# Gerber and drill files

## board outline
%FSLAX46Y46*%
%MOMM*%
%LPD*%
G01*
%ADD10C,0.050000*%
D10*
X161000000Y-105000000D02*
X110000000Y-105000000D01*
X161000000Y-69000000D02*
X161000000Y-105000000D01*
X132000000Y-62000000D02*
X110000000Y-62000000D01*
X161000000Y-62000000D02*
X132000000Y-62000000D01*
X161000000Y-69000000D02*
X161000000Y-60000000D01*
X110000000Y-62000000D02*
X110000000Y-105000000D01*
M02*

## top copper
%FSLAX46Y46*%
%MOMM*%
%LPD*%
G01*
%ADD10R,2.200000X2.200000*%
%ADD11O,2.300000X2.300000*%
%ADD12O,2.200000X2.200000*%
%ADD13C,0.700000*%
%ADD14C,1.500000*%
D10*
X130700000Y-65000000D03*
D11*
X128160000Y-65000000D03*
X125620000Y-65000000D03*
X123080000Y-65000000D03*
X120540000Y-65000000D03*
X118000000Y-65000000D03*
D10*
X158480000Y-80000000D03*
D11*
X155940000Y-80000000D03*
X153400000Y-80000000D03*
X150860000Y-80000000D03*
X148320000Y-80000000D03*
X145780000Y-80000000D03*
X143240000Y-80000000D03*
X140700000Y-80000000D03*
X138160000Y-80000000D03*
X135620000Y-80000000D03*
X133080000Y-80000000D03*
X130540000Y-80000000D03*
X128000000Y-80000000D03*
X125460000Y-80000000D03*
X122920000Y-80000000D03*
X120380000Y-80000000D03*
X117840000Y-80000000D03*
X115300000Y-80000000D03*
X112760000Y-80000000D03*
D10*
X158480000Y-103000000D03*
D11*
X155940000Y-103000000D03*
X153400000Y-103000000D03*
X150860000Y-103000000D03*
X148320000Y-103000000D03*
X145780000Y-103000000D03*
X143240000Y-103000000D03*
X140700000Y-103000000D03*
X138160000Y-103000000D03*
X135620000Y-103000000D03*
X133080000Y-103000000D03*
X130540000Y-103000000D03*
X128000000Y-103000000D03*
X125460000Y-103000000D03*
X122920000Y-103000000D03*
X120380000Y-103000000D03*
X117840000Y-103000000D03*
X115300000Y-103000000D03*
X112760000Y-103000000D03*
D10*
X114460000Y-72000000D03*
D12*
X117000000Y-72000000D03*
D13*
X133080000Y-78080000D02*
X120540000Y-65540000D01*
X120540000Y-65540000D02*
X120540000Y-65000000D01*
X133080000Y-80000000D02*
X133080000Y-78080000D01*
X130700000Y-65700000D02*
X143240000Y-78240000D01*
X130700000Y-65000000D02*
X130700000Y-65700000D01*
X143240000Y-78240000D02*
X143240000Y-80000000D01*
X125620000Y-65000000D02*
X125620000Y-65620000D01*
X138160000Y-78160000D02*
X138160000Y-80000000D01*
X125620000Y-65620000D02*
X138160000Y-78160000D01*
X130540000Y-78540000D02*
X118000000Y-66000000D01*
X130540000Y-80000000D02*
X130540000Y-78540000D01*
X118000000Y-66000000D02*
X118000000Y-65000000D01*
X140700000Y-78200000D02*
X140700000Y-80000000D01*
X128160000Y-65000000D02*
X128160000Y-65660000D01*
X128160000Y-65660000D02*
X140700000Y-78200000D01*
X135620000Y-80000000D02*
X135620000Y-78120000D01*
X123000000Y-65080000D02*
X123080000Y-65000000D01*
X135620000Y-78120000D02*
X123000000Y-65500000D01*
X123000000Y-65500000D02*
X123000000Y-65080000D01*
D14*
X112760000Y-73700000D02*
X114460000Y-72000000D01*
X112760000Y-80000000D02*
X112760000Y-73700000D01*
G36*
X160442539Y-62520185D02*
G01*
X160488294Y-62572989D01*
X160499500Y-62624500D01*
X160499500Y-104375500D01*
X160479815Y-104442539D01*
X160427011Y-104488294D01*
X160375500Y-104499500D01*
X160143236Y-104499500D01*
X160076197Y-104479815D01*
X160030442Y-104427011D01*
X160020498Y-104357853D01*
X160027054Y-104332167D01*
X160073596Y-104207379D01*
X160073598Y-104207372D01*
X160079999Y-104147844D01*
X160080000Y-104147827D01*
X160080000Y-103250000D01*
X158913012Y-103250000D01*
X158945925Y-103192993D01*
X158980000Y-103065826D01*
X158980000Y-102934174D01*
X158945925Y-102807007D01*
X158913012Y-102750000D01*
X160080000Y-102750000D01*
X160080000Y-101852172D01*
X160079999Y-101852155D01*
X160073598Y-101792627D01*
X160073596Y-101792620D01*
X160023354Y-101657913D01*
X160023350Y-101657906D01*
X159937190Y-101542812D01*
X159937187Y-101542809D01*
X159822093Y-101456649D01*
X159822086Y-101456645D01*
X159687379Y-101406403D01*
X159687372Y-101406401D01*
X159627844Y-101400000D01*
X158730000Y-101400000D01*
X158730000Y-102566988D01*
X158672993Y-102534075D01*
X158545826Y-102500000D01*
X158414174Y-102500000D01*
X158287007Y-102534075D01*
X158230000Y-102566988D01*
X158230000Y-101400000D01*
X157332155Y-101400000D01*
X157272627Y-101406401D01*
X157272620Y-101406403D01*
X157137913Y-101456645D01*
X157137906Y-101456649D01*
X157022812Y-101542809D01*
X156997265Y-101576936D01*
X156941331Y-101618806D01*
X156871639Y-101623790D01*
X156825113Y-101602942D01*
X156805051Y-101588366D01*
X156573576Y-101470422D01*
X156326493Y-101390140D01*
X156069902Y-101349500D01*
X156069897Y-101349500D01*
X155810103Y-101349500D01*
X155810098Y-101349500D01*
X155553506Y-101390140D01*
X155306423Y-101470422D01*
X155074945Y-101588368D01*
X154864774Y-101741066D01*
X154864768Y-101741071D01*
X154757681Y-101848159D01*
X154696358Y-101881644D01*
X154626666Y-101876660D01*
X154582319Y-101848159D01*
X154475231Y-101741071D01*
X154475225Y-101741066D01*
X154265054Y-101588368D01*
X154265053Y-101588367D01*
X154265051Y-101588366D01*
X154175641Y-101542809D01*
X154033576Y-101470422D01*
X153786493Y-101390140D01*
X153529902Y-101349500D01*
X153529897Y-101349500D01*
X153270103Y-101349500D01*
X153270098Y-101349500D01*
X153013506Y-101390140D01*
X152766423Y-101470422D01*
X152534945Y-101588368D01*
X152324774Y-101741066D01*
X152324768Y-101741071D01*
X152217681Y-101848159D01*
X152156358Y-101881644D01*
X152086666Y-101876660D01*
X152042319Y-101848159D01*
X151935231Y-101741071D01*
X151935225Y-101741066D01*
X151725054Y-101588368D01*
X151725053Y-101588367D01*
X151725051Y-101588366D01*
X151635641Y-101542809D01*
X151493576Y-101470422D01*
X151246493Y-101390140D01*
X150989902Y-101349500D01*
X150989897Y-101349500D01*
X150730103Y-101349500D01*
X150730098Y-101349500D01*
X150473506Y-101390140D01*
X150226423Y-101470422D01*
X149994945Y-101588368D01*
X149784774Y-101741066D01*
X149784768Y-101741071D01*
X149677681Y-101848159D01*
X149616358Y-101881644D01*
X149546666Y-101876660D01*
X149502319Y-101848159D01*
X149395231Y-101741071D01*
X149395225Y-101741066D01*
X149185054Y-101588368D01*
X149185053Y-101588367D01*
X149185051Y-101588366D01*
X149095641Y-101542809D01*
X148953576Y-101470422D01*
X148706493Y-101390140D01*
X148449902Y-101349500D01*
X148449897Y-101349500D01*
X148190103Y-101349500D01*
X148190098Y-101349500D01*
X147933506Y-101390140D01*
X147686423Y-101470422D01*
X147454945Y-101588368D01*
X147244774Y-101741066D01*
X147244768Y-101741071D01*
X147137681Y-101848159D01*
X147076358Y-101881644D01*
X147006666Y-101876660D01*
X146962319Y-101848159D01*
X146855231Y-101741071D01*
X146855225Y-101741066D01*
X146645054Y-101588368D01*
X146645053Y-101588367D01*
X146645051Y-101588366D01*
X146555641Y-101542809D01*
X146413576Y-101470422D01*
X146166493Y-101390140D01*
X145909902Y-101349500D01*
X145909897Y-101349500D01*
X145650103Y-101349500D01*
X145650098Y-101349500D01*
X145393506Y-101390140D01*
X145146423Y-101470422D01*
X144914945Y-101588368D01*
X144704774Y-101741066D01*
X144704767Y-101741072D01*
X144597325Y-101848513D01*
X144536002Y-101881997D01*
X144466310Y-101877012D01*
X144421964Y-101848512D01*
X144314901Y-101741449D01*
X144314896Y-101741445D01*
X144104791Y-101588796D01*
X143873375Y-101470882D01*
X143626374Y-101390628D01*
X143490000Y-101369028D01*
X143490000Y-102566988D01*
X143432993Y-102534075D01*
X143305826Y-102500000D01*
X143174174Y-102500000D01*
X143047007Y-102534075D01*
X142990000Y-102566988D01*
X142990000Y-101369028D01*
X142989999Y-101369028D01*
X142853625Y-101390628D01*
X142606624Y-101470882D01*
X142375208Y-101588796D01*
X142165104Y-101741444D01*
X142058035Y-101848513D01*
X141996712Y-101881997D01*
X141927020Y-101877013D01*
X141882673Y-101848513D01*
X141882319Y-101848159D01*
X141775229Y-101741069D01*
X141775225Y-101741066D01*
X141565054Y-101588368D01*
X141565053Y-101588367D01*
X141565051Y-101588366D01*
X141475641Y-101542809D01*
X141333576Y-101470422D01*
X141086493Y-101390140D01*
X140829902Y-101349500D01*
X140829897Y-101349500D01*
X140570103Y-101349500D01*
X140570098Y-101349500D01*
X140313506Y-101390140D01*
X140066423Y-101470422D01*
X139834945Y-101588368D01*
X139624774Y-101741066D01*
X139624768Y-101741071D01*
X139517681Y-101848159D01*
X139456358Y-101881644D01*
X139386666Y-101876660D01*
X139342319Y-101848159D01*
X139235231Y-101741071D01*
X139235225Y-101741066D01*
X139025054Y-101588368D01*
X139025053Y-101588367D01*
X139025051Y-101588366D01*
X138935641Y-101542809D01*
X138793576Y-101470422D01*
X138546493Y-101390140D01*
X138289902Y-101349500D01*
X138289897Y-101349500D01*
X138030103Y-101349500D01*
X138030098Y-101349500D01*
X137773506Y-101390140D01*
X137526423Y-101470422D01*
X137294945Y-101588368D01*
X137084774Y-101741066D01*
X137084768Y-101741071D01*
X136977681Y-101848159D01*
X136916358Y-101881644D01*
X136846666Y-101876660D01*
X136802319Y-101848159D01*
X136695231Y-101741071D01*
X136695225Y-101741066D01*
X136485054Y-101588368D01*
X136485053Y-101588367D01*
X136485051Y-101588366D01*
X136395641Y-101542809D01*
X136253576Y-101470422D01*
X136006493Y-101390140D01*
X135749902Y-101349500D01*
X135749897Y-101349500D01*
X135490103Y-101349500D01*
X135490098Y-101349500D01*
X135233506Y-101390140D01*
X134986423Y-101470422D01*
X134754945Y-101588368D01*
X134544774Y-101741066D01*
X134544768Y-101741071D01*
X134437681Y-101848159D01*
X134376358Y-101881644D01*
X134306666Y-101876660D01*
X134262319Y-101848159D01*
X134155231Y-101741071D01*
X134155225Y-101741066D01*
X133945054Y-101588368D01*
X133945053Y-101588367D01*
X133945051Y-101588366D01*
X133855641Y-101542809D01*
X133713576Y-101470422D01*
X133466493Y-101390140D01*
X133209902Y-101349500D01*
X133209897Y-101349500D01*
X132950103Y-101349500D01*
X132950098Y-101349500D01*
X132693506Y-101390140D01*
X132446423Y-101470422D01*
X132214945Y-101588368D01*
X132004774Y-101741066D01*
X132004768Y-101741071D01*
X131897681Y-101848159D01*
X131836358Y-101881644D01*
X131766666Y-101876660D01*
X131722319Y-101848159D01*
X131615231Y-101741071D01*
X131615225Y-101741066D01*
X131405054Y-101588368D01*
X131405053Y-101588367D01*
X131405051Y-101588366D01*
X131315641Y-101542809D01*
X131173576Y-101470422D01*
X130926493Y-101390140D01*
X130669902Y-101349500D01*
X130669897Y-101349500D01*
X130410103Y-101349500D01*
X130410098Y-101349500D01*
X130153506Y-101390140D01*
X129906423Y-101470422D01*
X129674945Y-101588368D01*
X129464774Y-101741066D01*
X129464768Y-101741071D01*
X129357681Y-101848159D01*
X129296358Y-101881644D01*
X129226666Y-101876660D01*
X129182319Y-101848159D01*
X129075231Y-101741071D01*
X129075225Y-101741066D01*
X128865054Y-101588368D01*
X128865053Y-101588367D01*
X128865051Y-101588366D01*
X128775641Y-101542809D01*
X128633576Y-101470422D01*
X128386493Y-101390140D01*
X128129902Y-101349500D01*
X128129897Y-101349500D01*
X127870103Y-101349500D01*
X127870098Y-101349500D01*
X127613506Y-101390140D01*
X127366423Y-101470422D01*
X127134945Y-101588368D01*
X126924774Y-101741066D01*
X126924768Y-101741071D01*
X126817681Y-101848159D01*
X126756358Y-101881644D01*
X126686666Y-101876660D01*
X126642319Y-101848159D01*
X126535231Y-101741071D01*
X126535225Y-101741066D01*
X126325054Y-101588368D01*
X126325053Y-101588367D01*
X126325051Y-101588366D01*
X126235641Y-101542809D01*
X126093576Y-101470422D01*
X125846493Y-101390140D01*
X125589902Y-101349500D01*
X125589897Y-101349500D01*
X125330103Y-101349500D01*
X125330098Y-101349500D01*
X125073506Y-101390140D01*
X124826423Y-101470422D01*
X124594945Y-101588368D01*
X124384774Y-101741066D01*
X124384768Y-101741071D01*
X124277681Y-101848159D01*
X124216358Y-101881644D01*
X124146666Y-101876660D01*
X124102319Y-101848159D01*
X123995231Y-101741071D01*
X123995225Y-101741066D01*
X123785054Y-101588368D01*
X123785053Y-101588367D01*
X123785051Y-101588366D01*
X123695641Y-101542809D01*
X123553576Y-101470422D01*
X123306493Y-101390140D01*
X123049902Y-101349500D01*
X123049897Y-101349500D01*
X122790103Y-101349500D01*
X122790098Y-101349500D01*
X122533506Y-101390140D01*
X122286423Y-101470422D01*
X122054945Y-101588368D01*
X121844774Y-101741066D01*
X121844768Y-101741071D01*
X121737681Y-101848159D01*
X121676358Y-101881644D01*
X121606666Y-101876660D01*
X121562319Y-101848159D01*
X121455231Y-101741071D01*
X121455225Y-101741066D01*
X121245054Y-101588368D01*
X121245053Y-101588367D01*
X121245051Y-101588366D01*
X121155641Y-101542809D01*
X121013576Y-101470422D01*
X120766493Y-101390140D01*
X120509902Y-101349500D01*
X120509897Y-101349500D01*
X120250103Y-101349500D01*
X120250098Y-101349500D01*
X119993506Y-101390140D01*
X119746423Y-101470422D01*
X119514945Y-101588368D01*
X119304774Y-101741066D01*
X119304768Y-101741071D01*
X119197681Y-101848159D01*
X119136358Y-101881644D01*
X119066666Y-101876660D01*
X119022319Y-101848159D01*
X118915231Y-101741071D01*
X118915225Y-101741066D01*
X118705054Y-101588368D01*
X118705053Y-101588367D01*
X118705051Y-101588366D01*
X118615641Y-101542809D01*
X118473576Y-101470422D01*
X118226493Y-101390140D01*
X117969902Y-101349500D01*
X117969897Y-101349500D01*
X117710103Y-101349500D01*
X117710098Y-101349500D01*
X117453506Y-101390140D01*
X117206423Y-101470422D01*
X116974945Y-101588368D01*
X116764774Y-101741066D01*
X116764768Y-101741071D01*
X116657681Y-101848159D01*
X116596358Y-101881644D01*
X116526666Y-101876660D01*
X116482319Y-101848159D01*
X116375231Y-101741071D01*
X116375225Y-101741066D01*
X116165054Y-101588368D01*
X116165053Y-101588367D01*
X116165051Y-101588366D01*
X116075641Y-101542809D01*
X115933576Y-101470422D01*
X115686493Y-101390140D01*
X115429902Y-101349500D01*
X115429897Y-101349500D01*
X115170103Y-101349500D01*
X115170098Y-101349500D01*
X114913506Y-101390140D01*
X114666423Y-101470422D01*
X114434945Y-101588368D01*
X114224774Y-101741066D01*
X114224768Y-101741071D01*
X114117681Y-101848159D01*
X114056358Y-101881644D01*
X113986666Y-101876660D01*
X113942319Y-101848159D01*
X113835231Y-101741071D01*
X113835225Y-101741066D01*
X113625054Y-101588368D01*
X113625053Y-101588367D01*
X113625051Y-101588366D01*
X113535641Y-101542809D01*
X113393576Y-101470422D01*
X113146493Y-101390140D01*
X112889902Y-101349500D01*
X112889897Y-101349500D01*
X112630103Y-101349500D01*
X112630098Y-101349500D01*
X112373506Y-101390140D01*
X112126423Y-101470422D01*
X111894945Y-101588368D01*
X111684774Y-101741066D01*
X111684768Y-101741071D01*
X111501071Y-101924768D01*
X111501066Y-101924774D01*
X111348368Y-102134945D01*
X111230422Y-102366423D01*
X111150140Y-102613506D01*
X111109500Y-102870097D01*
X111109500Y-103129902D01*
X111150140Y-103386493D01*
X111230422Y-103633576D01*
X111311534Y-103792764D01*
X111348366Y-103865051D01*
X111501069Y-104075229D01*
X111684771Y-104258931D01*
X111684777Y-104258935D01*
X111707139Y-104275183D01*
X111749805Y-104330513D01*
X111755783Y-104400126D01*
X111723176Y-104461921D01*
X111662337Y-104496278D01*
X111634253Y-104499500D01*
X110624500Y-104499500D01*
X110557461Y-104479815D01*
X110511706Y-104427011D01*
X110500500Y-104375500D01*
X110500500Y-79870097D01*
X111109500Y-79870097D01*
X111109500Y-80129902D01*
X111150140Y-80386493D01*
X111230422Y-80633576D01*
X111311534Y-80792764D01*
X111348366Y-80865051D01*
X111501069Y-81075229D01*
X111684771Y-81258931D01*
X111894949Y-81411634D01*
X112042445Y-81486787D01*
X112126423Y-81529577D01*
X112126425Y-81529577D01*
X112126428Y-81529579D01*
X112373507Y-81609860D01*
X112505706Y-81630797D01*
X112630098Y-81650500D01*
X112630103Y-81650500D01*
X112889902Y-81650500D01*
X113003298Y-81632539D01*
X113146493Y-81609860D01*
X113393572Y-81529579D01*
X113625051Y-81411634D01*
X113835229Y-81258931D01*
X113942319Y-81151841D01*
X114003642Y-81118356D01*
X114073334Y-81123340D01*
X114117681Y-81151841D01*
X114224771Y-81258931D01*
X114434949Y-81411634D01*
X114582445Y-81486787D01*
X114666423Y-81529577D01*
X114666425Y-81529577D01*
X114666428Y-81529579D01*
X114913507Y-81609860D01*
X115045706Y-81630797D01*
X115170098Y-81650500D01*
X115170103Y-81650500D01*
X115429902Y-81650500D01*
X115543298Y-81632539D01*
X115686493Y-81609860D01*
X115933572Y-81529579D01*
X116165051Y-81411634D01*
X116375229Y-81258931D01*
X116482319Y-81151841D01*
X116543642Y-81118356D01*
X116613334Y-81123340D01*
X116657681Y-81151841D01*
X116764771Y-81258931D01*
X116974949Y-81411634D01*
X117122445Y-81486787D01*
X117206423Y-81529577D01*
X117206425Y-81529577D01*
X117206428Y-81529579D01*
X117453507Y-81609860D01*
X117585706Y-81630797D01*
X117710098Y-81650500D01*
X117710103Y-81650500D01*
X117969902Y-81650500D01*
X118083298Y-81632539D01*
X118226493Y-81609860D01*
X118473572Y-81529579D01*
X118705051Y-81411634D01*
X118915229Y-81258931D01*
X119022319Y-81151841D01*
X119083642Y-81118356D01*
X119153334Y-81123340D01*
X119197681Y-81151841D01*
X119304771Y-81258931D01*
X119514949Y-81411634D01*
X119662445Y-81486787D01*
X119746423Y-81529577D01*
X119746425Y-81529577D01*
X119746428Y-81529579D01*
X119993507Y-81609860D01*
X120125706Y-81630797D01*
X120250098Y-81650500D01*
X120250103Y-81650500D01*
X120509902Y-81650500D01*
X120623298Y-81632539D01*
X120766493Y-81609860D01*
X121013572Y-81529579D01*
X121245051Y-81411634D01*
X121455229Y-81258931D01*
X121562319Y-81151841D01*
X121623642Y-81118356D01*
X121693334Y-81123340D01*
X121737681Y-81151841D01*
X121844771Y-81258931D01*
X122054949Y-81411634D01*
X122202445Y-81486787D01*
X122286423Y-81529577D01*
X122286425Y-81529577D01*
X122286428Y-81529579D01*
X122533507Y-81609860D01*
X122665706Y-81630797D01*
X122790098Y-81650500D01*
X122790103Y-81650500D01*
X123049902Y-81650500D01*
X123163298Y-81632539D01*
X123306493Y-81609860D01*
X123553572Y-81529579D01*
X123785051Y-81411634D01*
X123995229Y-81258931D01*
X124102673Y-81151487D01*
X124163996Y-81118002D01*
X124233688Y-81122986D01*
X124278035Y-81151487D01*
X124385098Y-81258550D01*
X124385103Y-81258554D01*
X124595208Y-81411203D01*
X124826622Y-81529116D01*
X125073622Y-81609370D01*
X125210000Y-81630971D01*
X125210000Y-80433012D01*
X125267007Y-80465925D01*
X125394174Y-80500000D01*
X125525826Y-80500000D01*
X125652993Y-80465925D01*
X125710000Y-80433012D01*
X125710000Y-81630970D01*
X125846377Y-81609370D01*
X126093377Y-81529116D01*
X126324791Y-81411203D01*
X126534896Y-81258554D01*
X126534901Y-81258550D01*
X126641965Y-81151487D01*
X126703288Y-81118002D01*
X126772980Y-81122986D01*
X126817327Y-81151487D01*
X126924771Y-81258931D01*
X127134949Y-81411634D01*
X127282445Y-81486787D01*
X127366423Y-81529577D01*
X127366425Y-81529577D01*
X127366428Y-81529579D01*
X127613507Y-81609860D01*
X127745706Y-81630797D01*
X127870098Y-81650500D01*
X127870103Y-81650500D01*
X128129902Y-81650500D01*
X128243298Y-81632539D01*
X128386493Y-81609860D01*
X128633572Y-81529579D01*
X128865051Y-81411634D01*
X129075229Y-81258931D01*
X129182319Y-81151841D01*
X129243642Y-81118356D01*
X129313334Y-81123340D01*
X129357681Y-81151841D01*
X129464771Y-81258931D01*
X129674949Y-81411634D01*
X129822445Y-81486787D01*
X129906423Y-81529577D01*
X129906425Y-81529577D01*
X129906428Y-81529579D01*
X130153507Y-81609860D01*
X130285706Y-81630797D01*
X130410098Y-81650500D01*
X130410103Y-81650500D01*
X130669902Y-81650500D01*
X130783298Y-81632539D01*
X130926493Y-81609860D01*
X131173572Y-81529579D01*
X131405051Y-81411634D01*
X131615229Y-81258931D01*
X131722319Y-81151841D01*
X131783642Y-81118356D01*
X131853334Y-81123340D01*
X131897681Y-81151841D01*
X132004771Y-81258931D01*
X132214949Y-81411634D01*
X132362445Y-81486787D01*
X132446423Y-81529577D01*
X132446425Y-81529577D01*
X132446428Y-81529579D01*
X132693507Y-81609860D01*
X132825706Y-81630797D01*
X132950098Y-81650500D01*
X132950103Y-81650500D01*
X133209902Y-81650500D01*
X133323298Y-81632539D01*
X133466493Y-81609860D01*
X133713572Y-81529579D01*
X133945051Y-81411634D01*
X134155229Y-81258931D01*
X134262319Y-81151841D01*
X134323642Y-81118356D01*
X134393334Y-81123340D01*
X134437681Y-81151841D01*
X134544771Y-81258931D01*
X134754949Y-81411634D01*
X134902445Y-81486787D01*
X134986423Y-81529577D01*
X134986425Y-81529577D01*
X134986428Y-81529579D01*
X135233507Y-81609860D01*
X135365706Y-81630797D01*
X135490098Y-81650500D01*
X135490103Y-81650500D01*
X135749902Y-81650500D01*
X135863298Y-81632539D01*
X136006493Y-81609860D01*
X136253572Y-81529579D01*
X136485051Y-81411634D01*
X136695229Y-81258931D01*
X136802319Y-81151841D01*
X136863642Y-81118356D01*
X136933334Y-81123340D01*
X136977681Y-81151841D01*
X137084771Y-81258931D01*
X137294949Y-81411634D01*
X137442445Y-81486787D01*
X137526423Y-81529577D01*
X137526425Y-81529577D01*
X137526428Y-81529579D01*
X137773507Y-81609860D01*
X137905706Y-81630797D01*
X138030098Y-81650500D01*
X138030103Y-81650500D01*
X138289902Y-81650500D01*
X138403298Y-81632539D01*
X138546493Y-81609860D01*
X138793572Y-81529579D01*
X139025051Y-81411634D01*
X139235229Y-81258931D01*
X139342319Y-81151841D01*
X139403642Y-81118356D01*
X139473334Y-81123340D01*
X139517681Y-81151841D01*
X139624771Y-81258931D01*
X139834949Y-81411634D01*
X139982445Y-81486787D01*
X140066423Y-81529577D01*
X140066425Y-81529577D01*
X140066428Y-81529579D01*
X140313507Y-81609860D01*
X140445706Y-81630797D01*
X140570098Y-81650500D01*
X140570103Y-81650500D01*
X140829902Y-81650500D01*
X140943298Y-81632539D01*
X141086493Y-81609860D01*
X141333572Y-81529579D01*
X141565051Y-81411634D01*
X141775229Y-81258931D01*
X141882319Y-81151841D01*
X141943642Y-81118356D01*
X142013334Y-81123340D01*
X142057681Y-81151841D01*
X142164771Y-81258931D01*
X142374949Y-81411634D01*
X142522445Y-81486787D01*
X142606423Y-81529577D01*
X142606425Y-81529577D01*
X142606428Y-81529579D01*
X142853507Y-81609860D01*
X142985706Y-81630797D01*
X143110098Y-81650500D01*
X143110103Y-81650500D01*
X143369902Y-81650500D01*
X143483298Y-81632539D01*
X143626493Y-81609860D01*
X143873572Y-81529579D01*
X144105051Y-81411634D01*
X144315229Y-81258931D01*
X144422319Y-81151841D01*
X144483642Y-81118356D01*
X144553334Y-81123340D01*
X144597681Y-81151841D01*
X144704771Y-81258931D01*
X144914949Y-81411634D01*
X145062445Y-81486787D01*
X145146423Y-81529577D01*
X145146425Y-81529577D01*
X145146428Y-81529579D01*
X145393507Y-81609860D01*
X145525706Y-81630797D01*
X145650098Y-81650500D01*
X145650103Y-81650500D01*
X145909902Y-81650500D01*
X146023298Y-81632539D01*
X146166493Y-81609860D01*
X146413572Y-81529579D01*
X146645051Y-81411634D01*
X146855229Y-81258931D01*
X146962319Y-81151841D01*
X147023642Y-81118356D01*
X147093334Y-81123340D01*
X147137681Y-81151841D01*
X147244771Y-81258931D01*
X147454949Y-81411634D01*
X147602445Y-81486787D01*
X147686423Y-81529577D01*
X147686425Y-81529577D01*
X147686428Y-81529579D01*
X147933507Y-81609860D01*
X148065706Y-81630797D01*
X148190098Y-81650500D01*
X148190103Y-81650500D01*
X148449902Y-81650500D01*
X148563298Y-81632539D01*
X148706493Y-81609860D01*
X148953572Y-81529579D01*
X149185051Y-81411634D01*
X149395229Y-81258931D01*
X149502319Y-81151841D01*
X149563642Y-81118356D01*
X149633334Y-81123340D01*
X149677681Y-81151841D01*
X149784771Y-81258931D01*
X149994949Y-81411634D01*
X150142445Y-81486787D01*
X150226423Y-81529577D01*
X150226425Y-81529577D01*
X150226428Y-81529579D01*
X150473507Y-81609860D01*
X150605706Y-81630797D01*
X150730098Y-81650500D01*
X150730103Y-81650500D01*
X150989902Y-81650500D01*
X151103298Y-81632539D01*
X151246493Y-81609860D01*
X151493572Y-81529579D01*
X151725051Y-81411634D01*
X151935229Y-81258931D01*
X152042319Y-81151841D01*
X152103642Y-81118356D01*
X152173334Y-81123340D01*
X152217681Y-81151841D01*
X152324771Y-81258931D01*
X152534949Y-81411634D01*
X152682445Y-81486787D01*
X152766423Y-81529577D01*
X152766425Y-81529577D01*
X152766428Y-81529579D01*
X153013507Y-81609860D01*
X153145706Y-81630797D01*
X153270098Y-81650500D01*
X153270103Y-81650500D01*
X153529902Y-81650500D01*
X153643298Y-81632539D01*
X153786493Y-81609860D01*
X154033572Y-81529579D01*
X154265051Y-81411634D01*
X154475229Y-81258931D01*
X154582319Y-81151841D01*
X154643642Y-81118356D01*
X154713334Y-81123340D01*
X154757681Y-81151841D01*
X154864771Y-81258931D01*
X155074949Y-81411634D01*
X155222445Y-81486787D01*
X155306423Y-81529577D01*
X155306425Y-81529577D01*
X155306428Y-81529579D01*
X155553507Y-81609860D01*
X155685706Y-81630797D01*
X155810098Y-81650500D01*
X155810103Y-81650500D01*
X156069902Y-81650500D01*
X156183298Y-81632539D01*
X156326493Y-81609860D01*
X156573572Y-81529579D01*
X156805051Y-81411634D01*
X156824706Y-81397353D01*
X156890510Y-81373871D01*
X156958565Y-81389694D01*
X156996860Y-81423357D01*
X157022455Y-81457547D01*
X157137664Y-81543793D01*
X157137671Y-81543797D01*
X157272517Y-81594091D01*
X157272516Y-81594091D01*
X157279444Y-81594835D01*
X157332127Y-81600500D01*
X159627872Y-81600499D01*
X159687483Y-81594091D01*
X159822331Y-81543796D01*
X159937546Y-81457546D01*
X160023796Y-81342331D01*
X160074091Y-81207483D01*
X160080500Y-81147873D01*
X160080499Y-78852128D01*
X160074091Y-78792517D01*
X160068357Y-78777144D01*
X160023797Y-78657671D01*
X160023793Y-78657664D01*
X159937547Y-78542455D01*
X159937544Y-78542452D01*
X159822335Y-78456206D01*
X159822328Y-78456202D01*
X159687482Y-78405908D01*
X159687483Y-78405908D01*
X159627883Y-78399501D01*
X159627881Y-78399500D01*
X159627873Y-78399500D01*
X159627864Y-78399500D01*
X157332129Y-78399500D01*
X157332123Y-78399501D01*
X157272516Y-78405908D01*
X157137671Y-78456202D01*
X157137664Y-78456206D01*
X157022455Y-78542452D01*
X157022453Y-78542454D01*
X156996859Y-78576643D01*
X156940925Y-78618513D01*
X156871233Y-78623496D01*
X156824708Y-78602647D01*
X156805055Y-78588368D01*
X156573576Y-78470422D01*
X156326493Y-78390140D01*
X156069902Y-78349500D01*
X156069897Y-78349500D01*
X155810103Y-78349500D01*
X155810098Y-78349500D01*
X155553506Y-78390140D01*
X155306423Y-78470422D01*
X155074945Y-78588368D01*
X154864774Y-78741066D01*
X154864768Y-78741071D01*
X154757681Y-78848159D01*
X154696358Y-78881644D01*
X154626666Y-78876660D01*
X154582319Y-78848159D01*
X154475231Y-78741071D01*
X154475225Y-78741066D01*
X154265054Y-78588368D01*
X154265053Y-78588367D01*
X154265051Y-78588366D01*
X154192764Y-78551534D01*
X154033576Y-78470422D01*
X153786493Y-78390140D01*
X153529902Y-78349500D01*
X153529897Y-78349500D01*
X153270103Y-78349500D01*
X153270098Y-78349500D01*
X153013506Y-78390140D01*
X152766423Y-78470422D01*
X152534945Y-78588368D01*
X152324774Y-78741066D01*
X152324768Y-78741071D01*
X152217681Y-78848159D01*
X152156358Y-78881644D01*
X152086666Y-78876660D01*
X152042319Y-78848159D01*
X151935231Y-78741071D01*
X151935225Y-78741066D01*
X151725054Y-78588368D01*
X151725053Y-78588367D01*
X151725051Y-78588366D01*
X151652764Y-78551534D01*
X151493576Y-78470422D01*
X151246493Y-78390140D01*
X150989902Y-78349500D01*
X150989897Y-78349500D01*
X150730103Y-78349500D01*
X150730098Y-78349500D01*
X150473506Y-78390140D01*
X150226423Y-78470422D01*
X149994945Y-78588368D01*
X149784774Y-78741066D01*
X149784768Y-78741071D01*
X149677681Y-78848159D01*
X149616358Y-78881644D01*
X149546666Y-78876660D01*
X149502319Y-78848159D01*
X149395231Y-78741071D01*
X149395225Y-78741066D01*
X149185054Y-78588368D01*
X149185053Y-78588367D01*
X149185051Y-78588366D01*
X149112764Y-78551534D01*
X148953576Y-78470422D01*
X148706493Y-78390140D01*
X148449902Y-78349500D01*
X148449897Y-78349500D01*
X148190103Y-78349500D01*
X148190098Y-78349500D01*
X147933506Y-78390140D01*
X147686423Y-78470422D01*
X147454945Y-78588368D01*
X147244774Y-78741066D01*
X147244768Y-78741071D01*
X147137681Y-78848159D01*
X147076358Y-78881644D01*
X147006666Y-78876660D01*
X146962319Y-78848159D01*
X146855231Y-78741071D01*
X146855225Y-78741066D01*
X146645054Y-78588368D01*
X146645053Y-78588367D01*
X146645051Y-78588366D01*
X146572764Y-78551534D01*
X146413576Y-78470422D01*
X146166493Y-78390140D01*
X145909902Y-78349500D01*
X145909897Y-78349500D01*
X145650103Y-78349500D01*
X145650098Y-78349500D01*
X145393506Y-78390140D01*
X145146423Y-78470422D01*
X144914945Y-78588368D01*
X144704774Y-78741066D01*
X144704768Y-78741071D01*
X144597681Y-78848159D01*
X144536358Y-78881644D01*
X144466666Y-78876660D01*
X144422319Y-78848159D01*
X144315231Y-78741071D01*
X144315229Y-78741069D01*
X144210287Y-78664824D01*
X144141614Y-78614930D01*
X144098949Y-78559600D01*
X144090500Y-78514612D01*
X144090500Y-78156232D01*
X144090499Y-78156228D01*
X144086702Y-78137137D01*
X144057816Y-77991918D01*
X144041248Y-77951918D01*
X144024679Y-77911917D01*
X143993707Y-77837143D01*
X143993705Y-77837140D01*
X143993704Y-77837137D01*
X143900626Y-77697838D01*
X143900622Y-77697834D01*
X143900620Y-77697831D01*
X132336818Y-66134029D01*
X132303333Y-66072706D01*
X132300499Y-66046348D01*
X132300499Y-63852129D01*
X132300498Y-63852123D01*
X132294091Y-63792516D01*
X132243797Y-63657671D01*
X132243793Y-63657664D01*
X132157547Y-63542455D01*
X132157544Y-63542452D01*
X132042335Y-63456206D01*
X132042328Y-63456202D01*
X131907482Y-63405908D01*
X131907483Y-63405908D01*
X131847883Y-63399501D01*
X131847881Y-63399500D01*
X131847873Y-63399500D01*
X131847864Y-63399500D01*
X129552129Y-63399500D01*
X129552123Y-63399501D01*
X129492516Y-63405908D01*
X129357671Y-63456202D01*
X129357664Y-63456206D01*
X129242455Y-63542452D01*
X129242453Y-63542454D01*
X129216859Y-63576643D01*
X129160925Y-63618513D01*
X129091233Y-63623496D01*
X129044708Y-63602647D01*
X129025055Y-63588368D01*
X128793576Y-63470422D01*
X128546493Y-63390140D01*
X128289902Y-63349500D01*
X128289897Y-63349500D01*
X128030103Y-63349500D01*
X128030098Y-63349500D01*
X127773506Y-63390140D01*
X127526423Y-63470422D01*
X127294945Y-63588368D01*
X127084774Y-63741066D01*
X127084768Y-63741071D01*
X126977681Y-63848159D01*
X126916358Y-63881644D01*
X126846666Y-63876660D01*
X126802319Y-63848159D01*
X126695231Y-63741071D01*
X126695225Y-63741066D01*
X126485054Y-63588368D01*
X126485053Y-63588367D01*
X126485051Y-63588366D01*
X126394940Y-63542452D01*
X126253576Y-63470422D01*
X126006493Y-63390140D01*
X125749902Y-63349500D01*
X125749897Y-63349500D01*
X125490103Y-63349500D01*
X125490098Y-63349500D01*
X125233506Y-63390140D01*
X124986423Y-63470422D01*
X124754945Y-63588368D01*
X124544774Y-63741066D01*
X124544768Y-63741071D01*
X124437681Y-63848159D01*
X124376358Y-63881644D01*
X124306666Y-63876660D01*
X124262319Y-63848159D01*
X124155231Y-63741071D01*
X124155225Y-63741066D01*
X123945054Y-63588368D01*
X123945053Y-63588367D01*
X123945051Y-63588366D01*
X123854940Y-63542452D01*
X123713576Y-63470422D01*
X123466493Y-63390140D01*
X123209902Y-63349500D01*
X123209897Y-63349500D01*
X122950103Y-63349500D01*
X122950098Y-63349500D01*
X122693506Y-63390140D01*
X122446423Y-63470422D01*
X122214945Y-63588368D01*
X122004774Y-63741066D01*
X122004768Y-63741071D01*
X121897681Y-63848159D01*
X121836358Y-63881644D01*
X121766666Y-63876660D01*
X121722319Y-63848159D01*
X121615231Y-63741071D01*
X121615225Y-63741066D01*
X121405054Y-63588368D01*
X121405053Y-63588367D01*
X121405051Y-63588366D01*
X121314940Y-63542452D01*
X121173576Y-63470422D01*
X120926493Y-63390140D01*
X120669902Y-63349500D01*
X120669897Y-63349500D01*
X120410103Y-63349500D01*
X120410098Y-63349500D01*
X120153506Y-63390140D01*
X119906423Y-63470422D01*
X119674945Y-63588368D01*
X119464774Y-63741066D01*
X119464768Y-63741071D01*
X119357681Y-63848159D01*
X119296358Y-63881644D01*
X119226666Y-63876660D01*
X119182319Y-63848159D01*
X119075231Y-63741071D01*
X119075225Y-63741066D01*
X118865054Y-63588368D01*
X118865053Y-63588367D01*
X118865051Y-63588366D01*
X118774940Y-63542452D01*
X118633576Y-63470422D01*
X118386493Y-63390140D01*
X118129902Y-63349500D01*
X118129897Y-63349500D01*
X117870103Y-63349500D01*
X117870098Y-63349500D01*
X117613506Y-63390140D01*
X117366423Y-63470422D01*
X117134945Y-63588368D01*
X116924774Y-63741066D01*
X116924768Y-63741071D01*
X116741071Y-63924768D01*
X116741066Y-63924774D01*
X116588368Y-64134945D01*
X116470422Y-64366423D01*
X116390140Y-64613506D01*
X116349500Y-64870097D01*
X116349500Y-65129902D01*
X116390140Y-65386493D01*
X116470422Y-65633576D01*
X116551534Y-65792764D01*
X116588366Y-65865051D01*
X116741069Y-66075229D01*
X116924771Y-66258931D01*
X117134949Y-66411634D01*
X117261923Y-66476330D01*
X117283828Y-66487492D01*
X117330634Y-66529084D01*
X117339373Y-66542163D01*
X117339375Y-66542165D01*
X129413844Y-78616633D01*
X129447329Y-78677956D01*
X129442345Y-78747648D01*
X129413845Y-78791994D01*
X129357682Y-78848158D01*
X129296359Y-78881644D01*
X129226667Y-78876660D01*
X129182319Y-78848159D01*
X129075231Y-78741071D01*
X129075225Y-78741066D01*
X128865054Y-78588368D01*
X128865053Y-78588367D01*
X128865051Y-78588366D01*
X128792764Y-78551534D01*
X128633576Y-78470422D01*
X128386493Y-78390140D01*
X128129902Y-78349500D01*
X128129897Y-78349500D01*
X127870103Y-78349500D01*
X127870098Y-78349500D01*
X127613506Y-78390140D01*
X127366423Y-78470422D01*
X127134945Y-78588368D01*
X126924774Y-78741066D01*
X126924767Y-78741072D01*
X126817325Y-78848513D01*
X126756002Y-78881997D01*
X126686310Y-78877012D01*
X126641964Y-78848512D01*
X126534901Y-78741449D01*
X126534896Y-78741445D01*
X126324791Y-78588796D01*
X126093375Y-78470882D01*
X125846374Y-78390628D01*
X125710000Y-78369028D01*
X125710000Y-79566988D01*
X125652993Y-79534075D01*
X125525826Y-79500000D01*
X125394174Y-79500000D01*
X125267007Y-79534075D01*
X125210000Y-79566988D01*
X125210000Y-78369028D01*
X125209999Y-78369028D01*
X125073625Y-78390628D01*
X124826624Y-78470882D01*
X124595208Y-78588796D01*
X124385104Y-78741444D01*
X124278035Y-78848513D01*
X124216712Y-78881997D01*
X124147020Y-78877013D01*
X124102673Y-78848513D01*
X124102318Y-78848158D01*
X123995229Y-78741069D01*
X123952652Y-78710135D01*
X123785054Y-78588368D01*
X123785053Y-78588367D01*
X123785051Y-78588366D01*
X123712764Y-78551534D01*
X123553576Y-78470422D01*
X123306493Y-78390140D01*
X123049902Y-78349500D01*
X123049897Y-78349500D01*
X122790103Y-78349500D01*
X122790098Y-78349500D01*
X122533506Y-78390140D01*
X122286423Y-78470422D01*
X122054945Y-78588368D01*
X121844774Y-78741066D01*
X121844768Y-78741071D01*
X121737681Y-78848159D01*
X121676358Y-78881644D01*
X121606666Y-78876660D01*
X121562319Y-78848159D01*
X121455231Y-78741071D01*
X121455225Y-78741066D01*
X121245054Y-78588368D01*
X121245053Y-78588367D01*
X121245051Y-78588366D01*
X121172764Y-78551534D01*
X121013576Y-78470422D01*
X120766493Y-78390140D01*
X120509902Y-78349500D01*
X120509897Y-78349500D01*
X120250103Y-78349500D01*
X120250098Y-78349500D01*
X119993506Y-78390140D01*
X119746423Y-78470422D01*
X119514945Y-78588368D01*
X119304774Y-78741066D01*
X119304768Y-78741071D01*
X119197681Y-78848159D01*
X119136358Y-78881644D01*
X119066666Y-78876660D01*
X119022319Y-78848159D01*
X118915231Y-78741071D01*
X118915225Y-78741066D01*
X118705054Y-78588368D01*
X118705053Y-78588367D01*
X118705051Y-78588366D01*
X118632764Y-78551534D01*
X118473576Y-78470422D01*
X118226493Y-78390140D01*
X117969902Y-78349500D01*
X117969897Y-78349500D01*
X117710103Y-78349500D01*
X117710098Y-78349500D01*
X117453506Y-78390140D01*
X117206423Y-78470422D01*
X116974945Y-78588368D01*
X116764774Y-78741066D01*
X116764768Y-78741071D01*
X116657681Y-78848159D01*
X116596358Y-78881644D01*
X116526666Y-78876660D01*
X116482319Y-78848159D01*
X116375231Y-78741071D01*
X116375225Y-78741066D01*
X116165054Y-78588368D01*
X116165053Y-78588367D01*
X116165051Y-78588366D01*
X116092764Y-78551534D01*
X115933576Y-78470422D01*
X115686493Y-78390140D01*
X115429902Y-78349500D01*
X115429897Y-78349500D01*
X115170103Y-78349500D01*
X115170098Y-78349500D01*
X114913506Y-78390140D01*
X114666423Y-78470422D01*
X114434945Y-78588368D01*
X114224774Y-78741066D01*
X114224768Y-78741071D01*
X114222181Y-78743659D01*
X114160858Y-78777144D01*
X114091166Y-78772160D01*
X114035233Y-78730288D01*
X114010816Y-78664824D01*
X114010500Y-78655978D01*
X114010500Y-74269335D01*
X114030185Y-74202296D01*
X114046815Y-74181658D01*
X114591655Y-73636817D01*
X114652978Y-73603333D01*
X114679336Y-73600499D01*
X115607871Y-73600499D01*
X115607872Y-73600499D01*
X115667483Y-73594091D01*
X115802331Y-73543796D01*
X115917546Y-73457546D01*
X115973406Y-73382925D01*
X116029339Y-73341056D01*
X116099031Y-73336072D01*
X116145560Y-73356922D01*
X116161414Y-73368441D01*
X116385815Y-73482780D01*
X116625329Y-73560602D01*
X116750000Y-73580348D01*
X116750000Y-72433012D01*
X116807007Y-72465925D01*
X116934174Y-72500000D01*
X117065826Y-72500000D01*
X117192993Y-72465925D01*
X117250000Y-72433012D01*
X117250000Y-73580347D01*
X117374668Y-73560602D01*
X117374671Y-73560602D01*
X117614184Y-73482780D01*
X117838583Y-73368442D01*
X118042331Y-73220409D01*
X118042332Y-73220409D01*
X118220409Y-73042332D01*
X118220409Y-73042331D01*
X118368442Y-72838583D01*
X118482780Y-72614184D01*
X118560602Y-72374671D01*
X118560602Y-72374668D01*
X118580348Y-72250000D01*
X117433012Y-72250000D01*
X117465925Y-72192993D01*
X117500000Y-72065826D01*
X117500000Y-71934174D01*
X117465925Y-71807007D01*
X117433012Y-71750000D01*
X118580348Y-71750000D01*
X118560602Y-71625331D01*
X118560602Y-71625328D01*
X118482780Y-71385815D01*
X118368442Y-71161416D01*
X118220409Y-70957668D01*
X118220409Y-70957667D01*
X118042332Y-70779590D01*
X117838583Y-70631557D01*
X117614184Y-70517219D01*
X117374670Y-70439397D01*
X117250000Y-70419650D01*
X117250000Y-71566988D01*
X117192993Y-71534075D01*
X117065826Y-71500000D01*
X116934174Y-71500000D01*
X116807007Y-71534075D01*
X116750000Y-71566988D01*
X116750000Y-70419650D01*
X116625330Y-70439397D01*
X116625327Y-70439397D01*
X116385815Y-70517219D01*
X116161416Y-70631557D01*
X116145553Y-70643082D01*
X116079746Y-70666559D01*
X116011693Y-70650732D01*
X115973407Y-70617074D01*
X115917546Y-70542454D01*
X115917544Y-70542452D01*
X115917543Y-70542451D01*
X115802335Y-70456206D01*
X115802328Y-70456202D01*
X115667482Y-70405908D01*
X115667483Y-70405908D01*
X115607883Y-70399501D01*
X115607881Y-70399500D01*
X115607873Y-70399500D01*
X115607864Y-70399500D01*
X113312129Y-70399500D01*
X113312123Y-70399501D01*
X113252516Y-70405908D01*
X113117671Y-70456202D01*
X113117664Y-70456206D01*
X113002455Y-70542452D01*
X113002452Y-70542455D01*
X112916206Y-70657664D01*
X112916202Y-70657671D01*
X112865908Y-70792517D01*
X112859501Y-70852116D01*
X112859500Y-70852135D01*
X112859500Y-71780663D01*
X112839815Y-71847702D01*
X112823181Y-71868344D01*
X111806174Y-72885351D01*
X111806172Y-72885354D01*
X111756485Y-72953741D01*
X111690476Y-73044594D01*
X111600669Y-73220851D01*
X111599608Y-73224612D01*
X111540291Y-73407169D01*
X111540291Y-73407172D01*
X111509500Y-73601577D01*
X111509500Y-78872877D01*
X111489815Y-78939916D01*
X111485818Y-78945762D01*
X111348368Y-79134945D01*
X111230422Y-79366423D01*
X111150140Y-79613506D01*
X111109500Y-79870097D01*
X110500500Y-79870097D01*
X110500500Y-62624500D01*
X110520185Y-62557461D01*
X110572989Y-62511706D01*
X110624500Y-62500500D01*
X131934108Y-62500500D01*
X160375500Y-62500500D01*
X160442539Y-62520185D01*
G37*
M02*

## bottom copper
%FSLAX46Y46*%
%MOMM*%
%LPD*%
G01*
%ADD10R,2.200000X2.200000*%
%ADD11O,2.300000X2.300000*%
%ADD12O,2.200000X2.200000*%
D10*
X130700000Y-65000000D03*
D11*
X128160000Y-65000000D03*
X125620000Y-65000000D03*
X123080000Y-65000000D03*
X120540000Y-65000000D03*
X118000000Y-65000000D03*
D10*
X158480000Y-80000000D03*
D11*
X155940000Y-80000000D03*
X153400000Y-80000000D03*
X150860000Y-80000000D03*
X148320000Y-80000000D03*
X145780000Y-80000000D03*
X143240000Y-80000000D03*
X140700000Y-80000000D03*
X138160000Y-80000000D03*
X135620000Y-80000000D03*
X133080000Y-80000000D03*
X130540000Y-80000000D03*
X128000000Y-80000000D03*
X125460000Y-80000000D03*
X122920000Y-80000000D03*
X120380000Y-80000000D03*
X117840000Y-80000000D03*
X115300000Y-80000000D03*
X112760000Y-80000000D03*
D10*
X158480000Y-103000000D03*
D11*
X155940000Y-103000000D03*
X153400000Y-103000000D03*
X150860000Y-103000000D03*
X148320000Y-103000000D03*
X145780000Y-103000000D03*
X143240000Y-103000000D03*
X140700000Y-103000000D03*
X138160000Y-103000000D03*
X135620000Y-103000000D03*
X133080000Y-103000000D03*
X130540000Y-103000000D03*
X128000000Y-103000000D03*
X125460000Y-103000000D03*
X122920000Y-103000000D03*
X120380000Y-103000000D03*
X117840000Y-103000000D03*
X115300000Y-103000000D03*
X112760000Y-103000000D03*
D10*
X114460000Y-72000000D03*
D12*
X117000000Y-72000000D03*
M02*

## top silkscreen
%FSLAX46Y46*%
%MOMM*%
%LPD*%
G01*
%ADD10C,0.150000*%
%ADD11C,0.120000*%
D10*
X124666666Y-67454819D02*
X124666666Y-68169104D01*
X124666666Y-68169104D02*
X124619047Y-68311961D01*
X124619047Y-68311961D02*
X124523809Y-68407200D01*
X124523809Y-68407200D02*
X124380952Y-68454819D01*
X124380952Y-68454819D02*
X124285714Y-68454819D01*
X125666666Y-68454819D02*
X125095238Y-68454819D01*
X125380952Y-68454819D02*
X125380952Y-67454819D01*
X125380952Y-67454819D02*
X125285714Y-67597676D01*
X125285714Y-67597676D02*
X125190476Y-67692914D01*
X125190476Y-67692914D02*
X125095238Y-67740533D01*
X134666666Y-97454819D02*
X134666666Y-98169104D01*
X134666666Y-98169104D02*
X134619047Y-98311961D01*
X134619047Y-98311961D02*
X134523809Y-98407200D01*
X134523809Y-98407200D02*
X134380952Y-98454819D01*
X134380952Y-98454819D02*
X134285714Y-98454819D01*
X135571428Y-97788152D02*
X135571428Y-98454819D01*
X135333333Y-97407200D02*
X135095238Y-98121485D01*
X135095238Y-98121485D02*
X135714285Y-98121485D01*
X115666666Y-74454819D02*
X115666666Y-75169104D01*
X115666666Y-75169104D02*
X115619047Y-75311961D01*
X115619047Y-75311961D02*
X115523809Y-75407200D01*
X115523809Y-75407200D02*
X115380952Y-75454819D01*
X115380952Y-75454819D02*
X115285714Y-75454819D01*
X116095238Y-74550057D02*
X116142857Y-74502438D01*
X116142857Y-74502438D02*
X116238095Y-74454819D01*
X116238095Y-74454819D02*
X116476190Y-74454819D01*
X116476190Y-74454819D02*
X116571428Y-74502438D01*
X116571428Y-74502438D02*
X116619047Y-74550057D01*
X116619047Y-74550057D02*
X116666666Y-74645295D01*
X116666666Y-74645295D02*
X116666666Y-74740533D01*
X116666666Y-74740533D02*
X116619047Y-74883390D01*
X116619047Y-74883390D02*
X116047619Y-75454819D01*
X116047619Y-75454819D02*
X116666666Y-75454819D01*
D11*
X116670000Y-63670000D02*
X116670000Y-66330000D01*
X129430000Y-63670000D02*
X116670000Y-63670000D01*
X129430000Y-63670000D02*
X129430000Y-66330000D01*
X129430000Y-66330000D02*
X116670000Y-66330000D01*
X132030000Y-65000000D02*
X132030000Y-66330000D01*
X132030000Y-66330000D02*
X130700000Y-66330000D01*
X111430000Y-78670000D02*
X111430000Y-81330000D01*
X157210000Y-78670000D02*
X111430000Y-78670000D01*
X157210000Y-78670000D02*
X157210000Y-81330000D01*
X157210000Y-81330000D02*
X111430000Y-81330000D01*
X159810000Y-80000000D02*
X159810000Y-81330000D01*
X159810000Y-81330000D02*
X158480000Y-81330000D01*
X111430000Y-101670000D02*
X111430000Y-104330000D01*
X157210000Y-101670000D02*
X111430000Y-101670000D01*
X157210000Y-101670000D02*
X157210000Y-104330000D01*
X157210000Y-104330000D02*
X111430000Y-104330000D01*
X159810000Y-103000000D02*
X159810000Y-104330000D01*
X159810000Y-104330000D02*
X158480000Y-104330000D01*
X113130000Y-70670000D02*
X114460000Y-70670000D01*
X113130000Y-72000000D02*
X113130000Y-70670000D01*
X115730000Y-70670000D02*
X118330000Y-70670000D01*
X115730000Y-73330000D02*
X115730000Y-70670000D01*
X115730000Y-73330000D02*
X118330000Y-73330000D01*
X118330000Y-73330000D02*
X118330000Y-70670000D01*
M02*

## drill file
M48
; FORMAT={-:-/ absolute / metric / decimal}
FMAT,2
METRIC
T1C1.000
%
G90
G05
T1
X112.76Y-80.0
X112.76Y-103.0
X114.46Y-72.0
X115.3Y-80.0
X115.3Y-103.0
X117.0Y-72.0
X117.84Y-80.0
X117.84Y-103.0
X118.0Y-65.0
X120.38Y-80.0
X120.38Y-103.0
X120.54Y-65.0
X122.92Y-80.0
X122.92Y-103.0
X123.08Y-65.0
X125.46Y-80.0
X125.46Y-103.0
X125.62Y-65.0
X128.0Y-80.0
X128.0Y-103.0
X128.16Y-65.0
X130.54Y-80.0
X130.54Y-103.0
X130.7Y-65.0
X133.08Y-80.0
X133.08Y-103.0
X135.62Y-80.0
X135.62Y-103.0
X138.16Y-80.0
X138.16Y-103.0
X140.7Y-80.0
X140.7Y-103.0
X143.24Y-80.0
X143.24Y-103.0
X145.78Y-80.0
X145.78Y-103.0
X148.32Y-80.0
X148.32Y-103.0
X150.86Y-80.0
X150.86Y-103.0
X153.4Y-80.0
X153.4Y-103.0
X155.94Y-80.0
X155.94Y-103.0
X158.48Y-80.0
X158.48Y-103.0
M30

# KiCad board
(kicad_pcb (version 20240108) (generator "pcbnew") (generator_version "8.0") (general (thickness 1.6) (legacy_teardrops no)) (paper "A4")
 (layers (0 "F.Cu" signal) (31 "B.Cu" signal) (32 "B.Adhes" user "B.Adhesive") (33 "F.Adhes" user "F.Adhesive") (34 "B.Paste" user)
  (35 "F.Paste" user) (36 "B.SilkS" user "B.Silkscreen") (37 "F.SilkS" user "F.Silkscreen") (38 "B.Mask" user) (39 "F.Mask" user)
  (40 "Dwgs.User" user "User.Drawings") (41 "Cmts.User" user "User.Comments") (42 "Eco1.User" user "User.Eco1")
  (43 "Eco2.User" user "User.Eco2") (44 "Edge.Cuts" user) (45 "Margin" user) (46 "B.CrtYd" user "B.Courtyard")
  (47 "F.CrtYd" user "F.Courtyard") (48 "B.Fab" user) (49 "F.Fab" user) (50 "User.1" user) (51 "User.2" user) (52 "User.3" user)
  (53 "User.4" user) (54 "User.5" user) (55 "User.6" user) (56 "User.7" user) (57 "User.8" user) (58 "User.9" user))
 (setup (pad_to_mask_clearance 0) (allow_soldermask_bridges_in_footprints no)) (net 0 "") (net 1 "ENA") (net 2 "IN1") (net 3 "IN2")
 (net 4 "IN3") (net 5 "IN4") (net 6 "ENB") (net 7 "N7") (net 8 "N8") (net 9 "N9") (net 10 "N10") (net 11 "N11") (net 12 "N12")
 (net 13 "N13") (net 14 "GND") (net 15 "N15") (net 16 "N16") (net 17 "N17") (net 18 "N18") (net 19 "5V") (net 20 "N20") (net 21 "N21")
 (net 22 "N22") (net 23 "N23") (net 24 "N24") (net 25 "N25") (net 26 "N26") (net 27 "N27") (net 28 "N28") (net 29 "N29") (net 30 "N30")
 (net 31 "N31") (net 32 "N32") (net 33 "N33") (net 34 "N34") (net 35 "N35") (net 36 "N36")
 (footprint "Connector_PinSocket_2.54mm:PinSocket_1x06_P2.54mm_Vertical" (layer "F.Cu") (at 130.7 65 -90)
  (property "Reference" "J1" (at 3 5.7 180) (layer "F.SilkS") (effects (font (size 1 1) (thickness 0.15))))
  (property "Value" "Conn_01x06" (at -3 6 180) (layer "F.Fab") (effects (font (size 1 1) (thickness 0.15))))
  (fp_line (start -1.33 14.03) (end 1.33 14.03) (stroke (width 0.12) (type solid)) (layer "F.SilkS"))
  (fp_line (start -1.33 1.27) (end -1.33 14.03) (stroke (width 0.12) (type solid)) (layer "F.SilkS"))
  (fp_line (start -1.33 1.27) (end 1.33 1.27) (stroke (width 0.12) (type solid)) (layer "F.SilkS"))
  (fp_line (start 1.33 1.27) (end 1.33 14.03) (stroke (width 0.12) (type solid)) (layer "F.SilkS"))
  (fp_line (start 0 -1.33) (end 1.33 -1.33) (stroke (width 0.12) (type solid)) (layer "F.SilkS"))
  (fp_line (start 1.33 -1.33) (end 1.33 0) (stroke (width 0.12) (type solid)) (layer "F.SilkS"))
  (pad "1" thru_hole rect (at 0 0 270) (size 2.2 2.2) (drill 1) (layers "*.Cu" "*.Mask") (remove_unused_layers no) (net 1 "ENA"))
  (pad "2" thru_hole oval (at 0 2.54 270) (size 2.3 2.3) (drill 1) (layers "*.Cu" "*.Mask") (remove_unused_layers no) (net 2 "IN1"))
  (pad "3" thru_hole oval (at 0 5.08 270) (size 2.3 2.3) (drill 1) (layers "*.Cu" "*.Mask") (remove_unused_layers no) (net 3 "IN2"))
  (pad "4" thru_hole oval (at 0 7.62 270) (size 2.3 2.3) (drill 1) (layers "*.Cu" "*.Mask") (remove_unused_layers no) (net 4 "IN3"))
  (pad "5" thru_hole oval (at 0 10.16 270) (size 2.3 2.3) (drill 1) (layers "*.Cu" "*.Mask") (remove_unused_layers no) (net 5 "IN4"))
  (pad "6" thru_hole oval (at 0 12.7 270) (size 2.3 2.3) (drill 1) (layers "*.Cu" "*.Mask") (remove_unused_layers no) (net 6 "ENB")))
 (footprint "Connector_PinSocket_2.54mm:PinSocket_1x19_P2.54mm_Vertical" (layer "F.Cu") (at 158.48 80 -90)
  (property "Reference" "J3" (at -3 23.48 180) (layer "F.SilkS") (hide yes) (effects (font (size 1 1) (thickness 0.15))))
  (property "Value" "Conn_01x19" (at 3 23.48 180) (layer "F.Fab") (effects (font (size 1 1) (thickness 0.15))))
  (fp_line (start -1.33 47.05) (end 1.33 47.05) (stroke (width 0.12) (type solid)) (layer "F.SilkS"))
  (fp_line (start -1.33 1.27) (end -1.33 47.05) (stroke (width 0.12) (type solid)) (layer "F.SilkS"))
  (fp_line (start -1.33 1.27) (end 1.33 1.27) (stroke (width 0.12) (type solid)) (layer "F.SilkS"))
  (fp_line (start 1.33 1.27) (end 1.33 47.05) (stroke (width 0.12) (type solid)) (layer "F.SilkS"))
  (fp_line (start 0 -1.33) (end 1.33 -1.33) (stroke (width 0.12) (type solid)) (layer "F.SilkS"))
  (fp_line (start 1.33 -1.33) (end 1.33 0) (stroke (width 0.12) (type solid)) (layer "F.SilkS"))
  (pad "1" thru_hole rect (at 0 0 270) (size 2.2 2.2) (drill 1) (layers "*.Cu" "*.Mask") (remove_unused_layers no) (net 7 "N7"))
  (pad "2" thru_hole oval (at 0 2.54 270) (size 2.3 2.3) (drill 1) (layers "*.Cu" "*.Mask") (remove_unused_layers no) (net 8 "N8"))
  (pad "3" thru_hole oval (at 0 5.08 270) (size 2.3 2.3) (drill 1) (layers "*.Cu" "*.Mask") (remove_unused_layers no) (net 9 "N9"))
  (pad "4" thru_hole oval (at 0 7.62 270) (size 2.3 2.3) (drill 1) (layers "*.Cu" "*.Mask") (remove_unused_layers no) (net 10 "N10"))
  (pad "5" thru_hole oval (at 0 10.16 270) (size 2.3 2.3) (drill 1) (layers "*.Cu" "*.Mask") (remove_unused_layers no) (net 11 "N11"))
  (pad "6" thru_hole oval (at 0 12.7 270) (size 2.3 2.3) (drill 1) (layers "*.Cu" "*.Mask") (remove_unused_layers no) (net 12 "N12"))
  (pad "7" thru_hole oval (at 0 15.24 270) (size 2.3 2.3) (drill 1) (layers "*.Cu" "*.Mask") (remove_unused_layers no) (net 1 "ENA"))
  (pad "8" thru_hole oval (at 0 17.78 270) (size 2.3 2.3) (drill 1) (layers "*.Cu" "*.Mask") (remove_unused_layers no) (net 2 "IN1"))
  (pad "9" thru_hole oval (at 0 20.32 270) (size 2.3 2.3) (drill 1) (layers "*.Cu" "*.Mask") (remove_unused_layers no) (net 3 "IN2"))
  (pad "10" thru_hole oval (at 0 22.86 270) (size 2.3 2.3) (drill 1) (layers "*.Cu" "*.Mask") (remove_unused_layers no) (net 4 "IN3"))
  (pad "11" thru_hole oval (at 0 25.4 270) (size 2.3 2.3) (drill 1) (layers "*.Cu" "*.Mask") (remove_unused_layers no) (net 5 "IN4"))
  (pad "12" thru_hole oval (at 0 27.94 270) (size 2.3 2.3) (drill 1) (layers "*.Cu" "*.Mask") (remove_unused_layers no) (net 6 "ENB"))
  (pad "13" thru_hole oval (at 0 30.48 270) (size 2.3 2.3) (drill 1) (layers "*.Cu" "*.Mask") (remove_unused_layers no) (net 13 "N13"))
  (pad "14" thru_hole oval (at 0 33.02 270) (size 2.3 2.3) (drill 1) (layers "*.Cu" "*.Mask") (remove_unused_layers no) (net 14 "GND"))
  (pad "15" thru_hole oval (at 0 35.56 270) (size 2.3 2.3) (drill 1) (layers "*.Cu" "*.Mask") (remove_unused_layers no) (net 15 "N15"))
  (pad "16" thru_hole oval (at 0 38.1 270) (size 2.3 2.3) (drill 1) (layers "*.Cu" "*.Mask") (remove_unused_layers no) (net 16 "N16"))
  (pad "17" thru_hole oval (at 0 40.64 270) (size 2.3 2.3) (drill 1) (layers "*.Cu" "*.Mask") (remove_unused_layers no) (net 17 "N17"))
  (pad "18" thru_hole oval (at 0 43.18 270) (size 2.3 2.3) (drill 1) (layers "*.Cu" "*.Mask") (remove_unused_layers no) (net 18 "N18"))
  (pad "19" thru_hole oval (at 0 45.72 270) (size 2.3 2.3) (drill 1) (layers "*.Cu" "*.Mask") (remove_unused_layers no) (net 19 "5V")))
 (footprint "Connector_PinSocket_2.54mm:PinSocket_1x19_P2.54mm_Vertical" (layer "F.Cu") (at 158.48 103 -90)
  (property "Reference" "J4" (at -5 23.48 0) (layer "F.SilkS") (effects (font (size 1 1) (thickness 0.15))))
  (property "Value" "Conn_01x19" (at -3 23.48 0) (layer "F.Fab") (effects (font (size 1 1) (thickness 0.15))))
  (fp_line (start -1.33 47.05) (end 1.33 47.05) (stroke (width 0.12) (type solid)) (layer "F.SilkS"))
  (fp_line (start -1.33 1.27) (end -1.33 47.05) (stroke (width 0.12) (type solid)) (layer "F.SilkS"))
  (fp_line (start -1.33 1.27) (end 1.33 1.27) (stroke (width 0.12) (type solid)) (layer "F.SilkS"))
  (fp_line (start 1.33 1.27) (end 1.33 47.05) (stroke (width 0.12) (type solid)) (layer "F.SilkS"))
  (fp_line (start 0 -1.33) (end 1.33 -1.33) (stroke (width 0.12) (type solid)) (layer "F.SilkS"))
  (fp_line (start 1.33 -1.33) (end 1.33 0) (stroke (width 0.12) (type solid)) (layer "F.SilkS"))
  (pad "1" thru_hole rect (at 0 0 270) (size 2.2 2.2) (drill 1) (layers "*.Cu" "*.Mask") (remove_unused_layers no) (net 14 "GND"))
  (pad "2" thru_hole oval (at 0 2.54 270) (size 2.3 2.3) (drill 1) (layers "*.Cu" "*.Mask") (remove_unused_layers no) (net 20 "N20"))
  (pad "3" thru_hole oval (at 0 5.08 270) (size 2.3 2.3) (drill 1) (layers "*.Cu" "*.Mask") (remove_unused_layers no) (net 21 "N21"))
  (pad "4" thru_hole oval (at 0 7.62 270) (size 2.3 2.3) (drill 1) (layers "*.Cu" "*.Mask") (remove_unused_layers no) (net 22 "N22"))
  (pad "5" thru_hole oval (at 0 10.16 270) (size 2.3 2.3) (drill 1) (layers "*.Cu" "*.Mask") (remove_unused_layers no) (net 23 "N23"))
  (pad "6" thru_hole oval (at 0 12.7 270) (size 2.3 2.3) (drill 1) (layers "*.Cu" "*.Mask") (remove_unused_layers no) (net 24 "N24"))
  (pad "7" thru_hole oval (at 0 15.24 270) (size 2.3 2.3) (drill 1) (layers "*.Cu" "*.Mask") (remove_unused_layers no) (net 14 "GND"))
  (pad "8" thru_hole oval (at 0 17.78 270) (size 2.3 2.3) (drill 1) (layers "*.Cu" "*.Mask") (remove_unused_layers no) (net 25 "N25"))
  (pad "9" thru_hole oval (at 0 20.32 270) (size 2.3 2.3) (drill 1) (layers "*.Cu" "*.Mask") (remove_unused_layers no) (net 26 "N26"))
  (pad "10" thru_hole oval (at 0 22.86 270) (size 2.3 2.3) (drill 1) (layers "*.Cu" "*.Mask") (remove_unused_layers no) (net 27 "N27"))
  (pad "11" thru_hole oval (at 0 25.4 270) (size 2.3 2.3) (drill 1) (layers "*.Cu" "*.Mask") (remove_unused_layers no) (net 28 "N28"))
  (pad "12" thru_hole oval (at 0 27.94 270) (size 2.3 2.3) (drill 1) (layers "*.Cu" "*.Mask") (remove_unused_layers no) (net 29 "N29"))
  (pad "13" thru_hole oval (at 0 30.48 270) (size 2.3 2.3) (drill 1) (layers "*.Cu" "*.Mask") (remove_unused_layers no) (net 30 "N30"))
  (pad "14" thru_hole oval (at 0 33.02 270) (size 2.3 2.3) (drill 1) (layers "*.Cu" "*.Mask") (remove_unused_layers no) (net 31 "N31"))
  (pad "15" thru_hole oval (at 0 35.56 270) (size 2.3 2.3) (drill 1) (layers "*.Cu" "*.Mask") (remove_unused_layers no) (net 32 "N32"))
  (pad "16" thru_hole oval (at 0 38.1 270) (size 2.3 2.3) (drill 1) (layers "*.Cu" "*.Mask") (remove_unused_layers no) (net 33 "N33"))
  (pad "17" thru_hole oval (at 0 40.64 270) (size 2.3 2.3) (drill 1) (layers "*.Cu" "*.Mask") (remove_unused_layers no) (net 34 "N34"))
  (pad "18" thru_hole oval (at 0 43.18 270) (size 2.3 2.3) (drill 1) (layers "*.Cu" "*.Mask") (remove_unused_layers no) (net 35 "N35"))
  (pad "19" thru_hole oval (at 0 45.72 270) (size 2.3 2.3) (drill 1) (layers "*.Cu" "*.Mask") (remove_unused_layers no) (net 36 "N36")))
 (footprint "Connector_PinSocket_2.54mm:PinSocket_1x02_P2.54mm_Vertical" (layer "F.Cu") (at 114.46 72 90)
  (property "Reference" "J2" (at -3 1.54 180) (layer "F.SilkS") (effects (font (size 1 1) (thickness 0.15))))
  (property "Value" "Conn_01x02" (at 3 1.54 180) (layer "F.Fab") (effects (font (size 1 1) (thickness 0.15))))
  (fp_line (start 1.33 -1.33) (end 1.33 0) (stroke (width 0.12) (type solid)) (layer "F.SilkS"))
  (fp_line (start 0 -1.33) (end 1.33 -1.33) (stroke (width 0.12) (type solid)) (layer "F.SilkS"))
  (fp_line (start 1.33 1.27) (end 1.33 3.87) (stroke (width 0.12) (type solid)) (layer "F.SilkS"))
  (fp_line (start -1.33 1.27) (end 1.33 1.27) (stroke (width 0.12) (type solid)) (layer "F.SilkS"))
  (fp_line (start -1.33 1.27) (end -1.33 3.87) (stroke (width 0.12) (type solid)) (layer "F.SilkS"))
  (fp_line (start -1.33 3.87) (end 1.33 3.87) (stroke (width 0.12) (type solid)) (layer "F.SilkS"))
  (pad "1" thru_hole rect (at 0 0 90) (size 2.2 2.2) (drill 1) (layers "*.Cu" "*.Mask") (remove_unused_layers no) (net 19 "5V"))
  (pad "2" thru_hole oval (at 0 2.54 90) (size 2.2 2.2) (drill 1) (layers "*.Cu" "*.Mask") (remove_unused_layers no) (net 14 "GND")))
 (gr_line (start 161 105) (end 110 105) (stroke (width 0.05) (type default)) (layer "Edge.Cuts"))
 (gr_line (start 161 69) (end 161 105) (stroke (width 0.05) (type default)) (layer "Edge.Cuts"))
 (gr_line (start 132 62) (end 110 62) (stroke (width 0.05) (type default)) (layer "Edge.Cuts"))
 (gr_line (start 161 62) (end 132 62) (stroke (width 0.05) (type default)) (layer "Edge.Cuts"))
 (gr_line (start 161 69) (end 161 60) (stroke (width 0.05) (type default)) (layer "Edge.Cuts"))
 (gr_line (start 110 62) (end 110 105) (stroke (width 0.05) (type default)) (layer "Edge.Cuts"))
 (segment (start 133.08 78.08) (end 120.54 65.54) (width 0.7) (layer "F.Cu") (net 5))
 (segment (start 120.54 65.54) (end 120.54 65) (width 0.7) (layer "F.Cu") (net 5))
 (segment (start 133.08 80) (end 133.08 78.08) (width 0.7) (layer "F.Cu") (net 5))
 (segment (start 130.7 65.7) (end 143.24 78.24) (width 0.7) (layer "F.Cu") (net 1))
 (segment (start 130.7 65) (end 130.7 65.7) (width 0.7) (layer "F.Cu") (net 1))
 (segment (start 143.24 78.24) (end 143.24 80) (width 0.7) (layer "F.Cu") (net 1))
 (segment (start 125.62 65) (end 125.62 65.62) (width 0.7) (layer "F.Cu") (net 3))
 (segment (start 138.16 78.16) (end 138.16 80) (width 0.7) (layer "F.Cu") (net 3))
 (segment (start 125.62 65.62) (end 138.16 78.16) (width 0.7) (layer "F.Cu") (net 3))
 (segment (start 130.54 78.54) (end 118 66) (width 0.7) (layer "F.Cu") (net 6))
 (segment (start 130.54 80) (end 130.54 78.54) (width 0.7) (layer "F.Cu") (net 6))
 (segment (start 118 66) (end 118 65) (width 0.7) (layer "F.Cu") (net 6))
 (segment (start 140.7 78.2) (end 140.7 80) (width 0.7) (layer "F.Cu") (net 2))
 (segment (start 128.16 65) (end 128.16 65.66) (width 0.7) (layer "F.Cu") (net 2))
 (segment (start 128.16 65.66) (end 140.7 78.2) (width 0.7) (layer "F.Cu") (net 2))
 (segment (start 135.62 80) (end 135.62 78.12) (width 0.7) (layer "F.Cu") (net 4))
 (segment (start 123 65.08) (end 123.08 65) (width 0.7) (layer "F.Cu") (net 4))
 (segment (start 135.62 78.12) (end 123 65.5) (width 0.7) (layer "F.Cu") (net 4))
 (segment (start 123 65.5) (end 123 65.08) (width 0.7) (layer "F.Cu") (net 4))
 (segment (start 112.76 73.7) (end 114.46 72) (width 1.5) (layer "F.Cu") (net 19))
 (segment (start 112.76 80) (end 112.76 73.7) (width 1.5) (layer "F.Cu") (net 19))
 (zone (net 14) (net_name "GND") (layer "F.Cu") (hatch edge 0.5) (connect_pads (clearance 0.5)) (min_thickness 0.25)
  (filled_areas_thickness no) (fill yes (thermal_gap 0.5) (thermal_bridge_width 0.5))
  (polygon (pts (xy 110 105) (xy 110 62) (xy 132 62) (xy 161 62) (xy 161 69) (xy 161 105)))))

